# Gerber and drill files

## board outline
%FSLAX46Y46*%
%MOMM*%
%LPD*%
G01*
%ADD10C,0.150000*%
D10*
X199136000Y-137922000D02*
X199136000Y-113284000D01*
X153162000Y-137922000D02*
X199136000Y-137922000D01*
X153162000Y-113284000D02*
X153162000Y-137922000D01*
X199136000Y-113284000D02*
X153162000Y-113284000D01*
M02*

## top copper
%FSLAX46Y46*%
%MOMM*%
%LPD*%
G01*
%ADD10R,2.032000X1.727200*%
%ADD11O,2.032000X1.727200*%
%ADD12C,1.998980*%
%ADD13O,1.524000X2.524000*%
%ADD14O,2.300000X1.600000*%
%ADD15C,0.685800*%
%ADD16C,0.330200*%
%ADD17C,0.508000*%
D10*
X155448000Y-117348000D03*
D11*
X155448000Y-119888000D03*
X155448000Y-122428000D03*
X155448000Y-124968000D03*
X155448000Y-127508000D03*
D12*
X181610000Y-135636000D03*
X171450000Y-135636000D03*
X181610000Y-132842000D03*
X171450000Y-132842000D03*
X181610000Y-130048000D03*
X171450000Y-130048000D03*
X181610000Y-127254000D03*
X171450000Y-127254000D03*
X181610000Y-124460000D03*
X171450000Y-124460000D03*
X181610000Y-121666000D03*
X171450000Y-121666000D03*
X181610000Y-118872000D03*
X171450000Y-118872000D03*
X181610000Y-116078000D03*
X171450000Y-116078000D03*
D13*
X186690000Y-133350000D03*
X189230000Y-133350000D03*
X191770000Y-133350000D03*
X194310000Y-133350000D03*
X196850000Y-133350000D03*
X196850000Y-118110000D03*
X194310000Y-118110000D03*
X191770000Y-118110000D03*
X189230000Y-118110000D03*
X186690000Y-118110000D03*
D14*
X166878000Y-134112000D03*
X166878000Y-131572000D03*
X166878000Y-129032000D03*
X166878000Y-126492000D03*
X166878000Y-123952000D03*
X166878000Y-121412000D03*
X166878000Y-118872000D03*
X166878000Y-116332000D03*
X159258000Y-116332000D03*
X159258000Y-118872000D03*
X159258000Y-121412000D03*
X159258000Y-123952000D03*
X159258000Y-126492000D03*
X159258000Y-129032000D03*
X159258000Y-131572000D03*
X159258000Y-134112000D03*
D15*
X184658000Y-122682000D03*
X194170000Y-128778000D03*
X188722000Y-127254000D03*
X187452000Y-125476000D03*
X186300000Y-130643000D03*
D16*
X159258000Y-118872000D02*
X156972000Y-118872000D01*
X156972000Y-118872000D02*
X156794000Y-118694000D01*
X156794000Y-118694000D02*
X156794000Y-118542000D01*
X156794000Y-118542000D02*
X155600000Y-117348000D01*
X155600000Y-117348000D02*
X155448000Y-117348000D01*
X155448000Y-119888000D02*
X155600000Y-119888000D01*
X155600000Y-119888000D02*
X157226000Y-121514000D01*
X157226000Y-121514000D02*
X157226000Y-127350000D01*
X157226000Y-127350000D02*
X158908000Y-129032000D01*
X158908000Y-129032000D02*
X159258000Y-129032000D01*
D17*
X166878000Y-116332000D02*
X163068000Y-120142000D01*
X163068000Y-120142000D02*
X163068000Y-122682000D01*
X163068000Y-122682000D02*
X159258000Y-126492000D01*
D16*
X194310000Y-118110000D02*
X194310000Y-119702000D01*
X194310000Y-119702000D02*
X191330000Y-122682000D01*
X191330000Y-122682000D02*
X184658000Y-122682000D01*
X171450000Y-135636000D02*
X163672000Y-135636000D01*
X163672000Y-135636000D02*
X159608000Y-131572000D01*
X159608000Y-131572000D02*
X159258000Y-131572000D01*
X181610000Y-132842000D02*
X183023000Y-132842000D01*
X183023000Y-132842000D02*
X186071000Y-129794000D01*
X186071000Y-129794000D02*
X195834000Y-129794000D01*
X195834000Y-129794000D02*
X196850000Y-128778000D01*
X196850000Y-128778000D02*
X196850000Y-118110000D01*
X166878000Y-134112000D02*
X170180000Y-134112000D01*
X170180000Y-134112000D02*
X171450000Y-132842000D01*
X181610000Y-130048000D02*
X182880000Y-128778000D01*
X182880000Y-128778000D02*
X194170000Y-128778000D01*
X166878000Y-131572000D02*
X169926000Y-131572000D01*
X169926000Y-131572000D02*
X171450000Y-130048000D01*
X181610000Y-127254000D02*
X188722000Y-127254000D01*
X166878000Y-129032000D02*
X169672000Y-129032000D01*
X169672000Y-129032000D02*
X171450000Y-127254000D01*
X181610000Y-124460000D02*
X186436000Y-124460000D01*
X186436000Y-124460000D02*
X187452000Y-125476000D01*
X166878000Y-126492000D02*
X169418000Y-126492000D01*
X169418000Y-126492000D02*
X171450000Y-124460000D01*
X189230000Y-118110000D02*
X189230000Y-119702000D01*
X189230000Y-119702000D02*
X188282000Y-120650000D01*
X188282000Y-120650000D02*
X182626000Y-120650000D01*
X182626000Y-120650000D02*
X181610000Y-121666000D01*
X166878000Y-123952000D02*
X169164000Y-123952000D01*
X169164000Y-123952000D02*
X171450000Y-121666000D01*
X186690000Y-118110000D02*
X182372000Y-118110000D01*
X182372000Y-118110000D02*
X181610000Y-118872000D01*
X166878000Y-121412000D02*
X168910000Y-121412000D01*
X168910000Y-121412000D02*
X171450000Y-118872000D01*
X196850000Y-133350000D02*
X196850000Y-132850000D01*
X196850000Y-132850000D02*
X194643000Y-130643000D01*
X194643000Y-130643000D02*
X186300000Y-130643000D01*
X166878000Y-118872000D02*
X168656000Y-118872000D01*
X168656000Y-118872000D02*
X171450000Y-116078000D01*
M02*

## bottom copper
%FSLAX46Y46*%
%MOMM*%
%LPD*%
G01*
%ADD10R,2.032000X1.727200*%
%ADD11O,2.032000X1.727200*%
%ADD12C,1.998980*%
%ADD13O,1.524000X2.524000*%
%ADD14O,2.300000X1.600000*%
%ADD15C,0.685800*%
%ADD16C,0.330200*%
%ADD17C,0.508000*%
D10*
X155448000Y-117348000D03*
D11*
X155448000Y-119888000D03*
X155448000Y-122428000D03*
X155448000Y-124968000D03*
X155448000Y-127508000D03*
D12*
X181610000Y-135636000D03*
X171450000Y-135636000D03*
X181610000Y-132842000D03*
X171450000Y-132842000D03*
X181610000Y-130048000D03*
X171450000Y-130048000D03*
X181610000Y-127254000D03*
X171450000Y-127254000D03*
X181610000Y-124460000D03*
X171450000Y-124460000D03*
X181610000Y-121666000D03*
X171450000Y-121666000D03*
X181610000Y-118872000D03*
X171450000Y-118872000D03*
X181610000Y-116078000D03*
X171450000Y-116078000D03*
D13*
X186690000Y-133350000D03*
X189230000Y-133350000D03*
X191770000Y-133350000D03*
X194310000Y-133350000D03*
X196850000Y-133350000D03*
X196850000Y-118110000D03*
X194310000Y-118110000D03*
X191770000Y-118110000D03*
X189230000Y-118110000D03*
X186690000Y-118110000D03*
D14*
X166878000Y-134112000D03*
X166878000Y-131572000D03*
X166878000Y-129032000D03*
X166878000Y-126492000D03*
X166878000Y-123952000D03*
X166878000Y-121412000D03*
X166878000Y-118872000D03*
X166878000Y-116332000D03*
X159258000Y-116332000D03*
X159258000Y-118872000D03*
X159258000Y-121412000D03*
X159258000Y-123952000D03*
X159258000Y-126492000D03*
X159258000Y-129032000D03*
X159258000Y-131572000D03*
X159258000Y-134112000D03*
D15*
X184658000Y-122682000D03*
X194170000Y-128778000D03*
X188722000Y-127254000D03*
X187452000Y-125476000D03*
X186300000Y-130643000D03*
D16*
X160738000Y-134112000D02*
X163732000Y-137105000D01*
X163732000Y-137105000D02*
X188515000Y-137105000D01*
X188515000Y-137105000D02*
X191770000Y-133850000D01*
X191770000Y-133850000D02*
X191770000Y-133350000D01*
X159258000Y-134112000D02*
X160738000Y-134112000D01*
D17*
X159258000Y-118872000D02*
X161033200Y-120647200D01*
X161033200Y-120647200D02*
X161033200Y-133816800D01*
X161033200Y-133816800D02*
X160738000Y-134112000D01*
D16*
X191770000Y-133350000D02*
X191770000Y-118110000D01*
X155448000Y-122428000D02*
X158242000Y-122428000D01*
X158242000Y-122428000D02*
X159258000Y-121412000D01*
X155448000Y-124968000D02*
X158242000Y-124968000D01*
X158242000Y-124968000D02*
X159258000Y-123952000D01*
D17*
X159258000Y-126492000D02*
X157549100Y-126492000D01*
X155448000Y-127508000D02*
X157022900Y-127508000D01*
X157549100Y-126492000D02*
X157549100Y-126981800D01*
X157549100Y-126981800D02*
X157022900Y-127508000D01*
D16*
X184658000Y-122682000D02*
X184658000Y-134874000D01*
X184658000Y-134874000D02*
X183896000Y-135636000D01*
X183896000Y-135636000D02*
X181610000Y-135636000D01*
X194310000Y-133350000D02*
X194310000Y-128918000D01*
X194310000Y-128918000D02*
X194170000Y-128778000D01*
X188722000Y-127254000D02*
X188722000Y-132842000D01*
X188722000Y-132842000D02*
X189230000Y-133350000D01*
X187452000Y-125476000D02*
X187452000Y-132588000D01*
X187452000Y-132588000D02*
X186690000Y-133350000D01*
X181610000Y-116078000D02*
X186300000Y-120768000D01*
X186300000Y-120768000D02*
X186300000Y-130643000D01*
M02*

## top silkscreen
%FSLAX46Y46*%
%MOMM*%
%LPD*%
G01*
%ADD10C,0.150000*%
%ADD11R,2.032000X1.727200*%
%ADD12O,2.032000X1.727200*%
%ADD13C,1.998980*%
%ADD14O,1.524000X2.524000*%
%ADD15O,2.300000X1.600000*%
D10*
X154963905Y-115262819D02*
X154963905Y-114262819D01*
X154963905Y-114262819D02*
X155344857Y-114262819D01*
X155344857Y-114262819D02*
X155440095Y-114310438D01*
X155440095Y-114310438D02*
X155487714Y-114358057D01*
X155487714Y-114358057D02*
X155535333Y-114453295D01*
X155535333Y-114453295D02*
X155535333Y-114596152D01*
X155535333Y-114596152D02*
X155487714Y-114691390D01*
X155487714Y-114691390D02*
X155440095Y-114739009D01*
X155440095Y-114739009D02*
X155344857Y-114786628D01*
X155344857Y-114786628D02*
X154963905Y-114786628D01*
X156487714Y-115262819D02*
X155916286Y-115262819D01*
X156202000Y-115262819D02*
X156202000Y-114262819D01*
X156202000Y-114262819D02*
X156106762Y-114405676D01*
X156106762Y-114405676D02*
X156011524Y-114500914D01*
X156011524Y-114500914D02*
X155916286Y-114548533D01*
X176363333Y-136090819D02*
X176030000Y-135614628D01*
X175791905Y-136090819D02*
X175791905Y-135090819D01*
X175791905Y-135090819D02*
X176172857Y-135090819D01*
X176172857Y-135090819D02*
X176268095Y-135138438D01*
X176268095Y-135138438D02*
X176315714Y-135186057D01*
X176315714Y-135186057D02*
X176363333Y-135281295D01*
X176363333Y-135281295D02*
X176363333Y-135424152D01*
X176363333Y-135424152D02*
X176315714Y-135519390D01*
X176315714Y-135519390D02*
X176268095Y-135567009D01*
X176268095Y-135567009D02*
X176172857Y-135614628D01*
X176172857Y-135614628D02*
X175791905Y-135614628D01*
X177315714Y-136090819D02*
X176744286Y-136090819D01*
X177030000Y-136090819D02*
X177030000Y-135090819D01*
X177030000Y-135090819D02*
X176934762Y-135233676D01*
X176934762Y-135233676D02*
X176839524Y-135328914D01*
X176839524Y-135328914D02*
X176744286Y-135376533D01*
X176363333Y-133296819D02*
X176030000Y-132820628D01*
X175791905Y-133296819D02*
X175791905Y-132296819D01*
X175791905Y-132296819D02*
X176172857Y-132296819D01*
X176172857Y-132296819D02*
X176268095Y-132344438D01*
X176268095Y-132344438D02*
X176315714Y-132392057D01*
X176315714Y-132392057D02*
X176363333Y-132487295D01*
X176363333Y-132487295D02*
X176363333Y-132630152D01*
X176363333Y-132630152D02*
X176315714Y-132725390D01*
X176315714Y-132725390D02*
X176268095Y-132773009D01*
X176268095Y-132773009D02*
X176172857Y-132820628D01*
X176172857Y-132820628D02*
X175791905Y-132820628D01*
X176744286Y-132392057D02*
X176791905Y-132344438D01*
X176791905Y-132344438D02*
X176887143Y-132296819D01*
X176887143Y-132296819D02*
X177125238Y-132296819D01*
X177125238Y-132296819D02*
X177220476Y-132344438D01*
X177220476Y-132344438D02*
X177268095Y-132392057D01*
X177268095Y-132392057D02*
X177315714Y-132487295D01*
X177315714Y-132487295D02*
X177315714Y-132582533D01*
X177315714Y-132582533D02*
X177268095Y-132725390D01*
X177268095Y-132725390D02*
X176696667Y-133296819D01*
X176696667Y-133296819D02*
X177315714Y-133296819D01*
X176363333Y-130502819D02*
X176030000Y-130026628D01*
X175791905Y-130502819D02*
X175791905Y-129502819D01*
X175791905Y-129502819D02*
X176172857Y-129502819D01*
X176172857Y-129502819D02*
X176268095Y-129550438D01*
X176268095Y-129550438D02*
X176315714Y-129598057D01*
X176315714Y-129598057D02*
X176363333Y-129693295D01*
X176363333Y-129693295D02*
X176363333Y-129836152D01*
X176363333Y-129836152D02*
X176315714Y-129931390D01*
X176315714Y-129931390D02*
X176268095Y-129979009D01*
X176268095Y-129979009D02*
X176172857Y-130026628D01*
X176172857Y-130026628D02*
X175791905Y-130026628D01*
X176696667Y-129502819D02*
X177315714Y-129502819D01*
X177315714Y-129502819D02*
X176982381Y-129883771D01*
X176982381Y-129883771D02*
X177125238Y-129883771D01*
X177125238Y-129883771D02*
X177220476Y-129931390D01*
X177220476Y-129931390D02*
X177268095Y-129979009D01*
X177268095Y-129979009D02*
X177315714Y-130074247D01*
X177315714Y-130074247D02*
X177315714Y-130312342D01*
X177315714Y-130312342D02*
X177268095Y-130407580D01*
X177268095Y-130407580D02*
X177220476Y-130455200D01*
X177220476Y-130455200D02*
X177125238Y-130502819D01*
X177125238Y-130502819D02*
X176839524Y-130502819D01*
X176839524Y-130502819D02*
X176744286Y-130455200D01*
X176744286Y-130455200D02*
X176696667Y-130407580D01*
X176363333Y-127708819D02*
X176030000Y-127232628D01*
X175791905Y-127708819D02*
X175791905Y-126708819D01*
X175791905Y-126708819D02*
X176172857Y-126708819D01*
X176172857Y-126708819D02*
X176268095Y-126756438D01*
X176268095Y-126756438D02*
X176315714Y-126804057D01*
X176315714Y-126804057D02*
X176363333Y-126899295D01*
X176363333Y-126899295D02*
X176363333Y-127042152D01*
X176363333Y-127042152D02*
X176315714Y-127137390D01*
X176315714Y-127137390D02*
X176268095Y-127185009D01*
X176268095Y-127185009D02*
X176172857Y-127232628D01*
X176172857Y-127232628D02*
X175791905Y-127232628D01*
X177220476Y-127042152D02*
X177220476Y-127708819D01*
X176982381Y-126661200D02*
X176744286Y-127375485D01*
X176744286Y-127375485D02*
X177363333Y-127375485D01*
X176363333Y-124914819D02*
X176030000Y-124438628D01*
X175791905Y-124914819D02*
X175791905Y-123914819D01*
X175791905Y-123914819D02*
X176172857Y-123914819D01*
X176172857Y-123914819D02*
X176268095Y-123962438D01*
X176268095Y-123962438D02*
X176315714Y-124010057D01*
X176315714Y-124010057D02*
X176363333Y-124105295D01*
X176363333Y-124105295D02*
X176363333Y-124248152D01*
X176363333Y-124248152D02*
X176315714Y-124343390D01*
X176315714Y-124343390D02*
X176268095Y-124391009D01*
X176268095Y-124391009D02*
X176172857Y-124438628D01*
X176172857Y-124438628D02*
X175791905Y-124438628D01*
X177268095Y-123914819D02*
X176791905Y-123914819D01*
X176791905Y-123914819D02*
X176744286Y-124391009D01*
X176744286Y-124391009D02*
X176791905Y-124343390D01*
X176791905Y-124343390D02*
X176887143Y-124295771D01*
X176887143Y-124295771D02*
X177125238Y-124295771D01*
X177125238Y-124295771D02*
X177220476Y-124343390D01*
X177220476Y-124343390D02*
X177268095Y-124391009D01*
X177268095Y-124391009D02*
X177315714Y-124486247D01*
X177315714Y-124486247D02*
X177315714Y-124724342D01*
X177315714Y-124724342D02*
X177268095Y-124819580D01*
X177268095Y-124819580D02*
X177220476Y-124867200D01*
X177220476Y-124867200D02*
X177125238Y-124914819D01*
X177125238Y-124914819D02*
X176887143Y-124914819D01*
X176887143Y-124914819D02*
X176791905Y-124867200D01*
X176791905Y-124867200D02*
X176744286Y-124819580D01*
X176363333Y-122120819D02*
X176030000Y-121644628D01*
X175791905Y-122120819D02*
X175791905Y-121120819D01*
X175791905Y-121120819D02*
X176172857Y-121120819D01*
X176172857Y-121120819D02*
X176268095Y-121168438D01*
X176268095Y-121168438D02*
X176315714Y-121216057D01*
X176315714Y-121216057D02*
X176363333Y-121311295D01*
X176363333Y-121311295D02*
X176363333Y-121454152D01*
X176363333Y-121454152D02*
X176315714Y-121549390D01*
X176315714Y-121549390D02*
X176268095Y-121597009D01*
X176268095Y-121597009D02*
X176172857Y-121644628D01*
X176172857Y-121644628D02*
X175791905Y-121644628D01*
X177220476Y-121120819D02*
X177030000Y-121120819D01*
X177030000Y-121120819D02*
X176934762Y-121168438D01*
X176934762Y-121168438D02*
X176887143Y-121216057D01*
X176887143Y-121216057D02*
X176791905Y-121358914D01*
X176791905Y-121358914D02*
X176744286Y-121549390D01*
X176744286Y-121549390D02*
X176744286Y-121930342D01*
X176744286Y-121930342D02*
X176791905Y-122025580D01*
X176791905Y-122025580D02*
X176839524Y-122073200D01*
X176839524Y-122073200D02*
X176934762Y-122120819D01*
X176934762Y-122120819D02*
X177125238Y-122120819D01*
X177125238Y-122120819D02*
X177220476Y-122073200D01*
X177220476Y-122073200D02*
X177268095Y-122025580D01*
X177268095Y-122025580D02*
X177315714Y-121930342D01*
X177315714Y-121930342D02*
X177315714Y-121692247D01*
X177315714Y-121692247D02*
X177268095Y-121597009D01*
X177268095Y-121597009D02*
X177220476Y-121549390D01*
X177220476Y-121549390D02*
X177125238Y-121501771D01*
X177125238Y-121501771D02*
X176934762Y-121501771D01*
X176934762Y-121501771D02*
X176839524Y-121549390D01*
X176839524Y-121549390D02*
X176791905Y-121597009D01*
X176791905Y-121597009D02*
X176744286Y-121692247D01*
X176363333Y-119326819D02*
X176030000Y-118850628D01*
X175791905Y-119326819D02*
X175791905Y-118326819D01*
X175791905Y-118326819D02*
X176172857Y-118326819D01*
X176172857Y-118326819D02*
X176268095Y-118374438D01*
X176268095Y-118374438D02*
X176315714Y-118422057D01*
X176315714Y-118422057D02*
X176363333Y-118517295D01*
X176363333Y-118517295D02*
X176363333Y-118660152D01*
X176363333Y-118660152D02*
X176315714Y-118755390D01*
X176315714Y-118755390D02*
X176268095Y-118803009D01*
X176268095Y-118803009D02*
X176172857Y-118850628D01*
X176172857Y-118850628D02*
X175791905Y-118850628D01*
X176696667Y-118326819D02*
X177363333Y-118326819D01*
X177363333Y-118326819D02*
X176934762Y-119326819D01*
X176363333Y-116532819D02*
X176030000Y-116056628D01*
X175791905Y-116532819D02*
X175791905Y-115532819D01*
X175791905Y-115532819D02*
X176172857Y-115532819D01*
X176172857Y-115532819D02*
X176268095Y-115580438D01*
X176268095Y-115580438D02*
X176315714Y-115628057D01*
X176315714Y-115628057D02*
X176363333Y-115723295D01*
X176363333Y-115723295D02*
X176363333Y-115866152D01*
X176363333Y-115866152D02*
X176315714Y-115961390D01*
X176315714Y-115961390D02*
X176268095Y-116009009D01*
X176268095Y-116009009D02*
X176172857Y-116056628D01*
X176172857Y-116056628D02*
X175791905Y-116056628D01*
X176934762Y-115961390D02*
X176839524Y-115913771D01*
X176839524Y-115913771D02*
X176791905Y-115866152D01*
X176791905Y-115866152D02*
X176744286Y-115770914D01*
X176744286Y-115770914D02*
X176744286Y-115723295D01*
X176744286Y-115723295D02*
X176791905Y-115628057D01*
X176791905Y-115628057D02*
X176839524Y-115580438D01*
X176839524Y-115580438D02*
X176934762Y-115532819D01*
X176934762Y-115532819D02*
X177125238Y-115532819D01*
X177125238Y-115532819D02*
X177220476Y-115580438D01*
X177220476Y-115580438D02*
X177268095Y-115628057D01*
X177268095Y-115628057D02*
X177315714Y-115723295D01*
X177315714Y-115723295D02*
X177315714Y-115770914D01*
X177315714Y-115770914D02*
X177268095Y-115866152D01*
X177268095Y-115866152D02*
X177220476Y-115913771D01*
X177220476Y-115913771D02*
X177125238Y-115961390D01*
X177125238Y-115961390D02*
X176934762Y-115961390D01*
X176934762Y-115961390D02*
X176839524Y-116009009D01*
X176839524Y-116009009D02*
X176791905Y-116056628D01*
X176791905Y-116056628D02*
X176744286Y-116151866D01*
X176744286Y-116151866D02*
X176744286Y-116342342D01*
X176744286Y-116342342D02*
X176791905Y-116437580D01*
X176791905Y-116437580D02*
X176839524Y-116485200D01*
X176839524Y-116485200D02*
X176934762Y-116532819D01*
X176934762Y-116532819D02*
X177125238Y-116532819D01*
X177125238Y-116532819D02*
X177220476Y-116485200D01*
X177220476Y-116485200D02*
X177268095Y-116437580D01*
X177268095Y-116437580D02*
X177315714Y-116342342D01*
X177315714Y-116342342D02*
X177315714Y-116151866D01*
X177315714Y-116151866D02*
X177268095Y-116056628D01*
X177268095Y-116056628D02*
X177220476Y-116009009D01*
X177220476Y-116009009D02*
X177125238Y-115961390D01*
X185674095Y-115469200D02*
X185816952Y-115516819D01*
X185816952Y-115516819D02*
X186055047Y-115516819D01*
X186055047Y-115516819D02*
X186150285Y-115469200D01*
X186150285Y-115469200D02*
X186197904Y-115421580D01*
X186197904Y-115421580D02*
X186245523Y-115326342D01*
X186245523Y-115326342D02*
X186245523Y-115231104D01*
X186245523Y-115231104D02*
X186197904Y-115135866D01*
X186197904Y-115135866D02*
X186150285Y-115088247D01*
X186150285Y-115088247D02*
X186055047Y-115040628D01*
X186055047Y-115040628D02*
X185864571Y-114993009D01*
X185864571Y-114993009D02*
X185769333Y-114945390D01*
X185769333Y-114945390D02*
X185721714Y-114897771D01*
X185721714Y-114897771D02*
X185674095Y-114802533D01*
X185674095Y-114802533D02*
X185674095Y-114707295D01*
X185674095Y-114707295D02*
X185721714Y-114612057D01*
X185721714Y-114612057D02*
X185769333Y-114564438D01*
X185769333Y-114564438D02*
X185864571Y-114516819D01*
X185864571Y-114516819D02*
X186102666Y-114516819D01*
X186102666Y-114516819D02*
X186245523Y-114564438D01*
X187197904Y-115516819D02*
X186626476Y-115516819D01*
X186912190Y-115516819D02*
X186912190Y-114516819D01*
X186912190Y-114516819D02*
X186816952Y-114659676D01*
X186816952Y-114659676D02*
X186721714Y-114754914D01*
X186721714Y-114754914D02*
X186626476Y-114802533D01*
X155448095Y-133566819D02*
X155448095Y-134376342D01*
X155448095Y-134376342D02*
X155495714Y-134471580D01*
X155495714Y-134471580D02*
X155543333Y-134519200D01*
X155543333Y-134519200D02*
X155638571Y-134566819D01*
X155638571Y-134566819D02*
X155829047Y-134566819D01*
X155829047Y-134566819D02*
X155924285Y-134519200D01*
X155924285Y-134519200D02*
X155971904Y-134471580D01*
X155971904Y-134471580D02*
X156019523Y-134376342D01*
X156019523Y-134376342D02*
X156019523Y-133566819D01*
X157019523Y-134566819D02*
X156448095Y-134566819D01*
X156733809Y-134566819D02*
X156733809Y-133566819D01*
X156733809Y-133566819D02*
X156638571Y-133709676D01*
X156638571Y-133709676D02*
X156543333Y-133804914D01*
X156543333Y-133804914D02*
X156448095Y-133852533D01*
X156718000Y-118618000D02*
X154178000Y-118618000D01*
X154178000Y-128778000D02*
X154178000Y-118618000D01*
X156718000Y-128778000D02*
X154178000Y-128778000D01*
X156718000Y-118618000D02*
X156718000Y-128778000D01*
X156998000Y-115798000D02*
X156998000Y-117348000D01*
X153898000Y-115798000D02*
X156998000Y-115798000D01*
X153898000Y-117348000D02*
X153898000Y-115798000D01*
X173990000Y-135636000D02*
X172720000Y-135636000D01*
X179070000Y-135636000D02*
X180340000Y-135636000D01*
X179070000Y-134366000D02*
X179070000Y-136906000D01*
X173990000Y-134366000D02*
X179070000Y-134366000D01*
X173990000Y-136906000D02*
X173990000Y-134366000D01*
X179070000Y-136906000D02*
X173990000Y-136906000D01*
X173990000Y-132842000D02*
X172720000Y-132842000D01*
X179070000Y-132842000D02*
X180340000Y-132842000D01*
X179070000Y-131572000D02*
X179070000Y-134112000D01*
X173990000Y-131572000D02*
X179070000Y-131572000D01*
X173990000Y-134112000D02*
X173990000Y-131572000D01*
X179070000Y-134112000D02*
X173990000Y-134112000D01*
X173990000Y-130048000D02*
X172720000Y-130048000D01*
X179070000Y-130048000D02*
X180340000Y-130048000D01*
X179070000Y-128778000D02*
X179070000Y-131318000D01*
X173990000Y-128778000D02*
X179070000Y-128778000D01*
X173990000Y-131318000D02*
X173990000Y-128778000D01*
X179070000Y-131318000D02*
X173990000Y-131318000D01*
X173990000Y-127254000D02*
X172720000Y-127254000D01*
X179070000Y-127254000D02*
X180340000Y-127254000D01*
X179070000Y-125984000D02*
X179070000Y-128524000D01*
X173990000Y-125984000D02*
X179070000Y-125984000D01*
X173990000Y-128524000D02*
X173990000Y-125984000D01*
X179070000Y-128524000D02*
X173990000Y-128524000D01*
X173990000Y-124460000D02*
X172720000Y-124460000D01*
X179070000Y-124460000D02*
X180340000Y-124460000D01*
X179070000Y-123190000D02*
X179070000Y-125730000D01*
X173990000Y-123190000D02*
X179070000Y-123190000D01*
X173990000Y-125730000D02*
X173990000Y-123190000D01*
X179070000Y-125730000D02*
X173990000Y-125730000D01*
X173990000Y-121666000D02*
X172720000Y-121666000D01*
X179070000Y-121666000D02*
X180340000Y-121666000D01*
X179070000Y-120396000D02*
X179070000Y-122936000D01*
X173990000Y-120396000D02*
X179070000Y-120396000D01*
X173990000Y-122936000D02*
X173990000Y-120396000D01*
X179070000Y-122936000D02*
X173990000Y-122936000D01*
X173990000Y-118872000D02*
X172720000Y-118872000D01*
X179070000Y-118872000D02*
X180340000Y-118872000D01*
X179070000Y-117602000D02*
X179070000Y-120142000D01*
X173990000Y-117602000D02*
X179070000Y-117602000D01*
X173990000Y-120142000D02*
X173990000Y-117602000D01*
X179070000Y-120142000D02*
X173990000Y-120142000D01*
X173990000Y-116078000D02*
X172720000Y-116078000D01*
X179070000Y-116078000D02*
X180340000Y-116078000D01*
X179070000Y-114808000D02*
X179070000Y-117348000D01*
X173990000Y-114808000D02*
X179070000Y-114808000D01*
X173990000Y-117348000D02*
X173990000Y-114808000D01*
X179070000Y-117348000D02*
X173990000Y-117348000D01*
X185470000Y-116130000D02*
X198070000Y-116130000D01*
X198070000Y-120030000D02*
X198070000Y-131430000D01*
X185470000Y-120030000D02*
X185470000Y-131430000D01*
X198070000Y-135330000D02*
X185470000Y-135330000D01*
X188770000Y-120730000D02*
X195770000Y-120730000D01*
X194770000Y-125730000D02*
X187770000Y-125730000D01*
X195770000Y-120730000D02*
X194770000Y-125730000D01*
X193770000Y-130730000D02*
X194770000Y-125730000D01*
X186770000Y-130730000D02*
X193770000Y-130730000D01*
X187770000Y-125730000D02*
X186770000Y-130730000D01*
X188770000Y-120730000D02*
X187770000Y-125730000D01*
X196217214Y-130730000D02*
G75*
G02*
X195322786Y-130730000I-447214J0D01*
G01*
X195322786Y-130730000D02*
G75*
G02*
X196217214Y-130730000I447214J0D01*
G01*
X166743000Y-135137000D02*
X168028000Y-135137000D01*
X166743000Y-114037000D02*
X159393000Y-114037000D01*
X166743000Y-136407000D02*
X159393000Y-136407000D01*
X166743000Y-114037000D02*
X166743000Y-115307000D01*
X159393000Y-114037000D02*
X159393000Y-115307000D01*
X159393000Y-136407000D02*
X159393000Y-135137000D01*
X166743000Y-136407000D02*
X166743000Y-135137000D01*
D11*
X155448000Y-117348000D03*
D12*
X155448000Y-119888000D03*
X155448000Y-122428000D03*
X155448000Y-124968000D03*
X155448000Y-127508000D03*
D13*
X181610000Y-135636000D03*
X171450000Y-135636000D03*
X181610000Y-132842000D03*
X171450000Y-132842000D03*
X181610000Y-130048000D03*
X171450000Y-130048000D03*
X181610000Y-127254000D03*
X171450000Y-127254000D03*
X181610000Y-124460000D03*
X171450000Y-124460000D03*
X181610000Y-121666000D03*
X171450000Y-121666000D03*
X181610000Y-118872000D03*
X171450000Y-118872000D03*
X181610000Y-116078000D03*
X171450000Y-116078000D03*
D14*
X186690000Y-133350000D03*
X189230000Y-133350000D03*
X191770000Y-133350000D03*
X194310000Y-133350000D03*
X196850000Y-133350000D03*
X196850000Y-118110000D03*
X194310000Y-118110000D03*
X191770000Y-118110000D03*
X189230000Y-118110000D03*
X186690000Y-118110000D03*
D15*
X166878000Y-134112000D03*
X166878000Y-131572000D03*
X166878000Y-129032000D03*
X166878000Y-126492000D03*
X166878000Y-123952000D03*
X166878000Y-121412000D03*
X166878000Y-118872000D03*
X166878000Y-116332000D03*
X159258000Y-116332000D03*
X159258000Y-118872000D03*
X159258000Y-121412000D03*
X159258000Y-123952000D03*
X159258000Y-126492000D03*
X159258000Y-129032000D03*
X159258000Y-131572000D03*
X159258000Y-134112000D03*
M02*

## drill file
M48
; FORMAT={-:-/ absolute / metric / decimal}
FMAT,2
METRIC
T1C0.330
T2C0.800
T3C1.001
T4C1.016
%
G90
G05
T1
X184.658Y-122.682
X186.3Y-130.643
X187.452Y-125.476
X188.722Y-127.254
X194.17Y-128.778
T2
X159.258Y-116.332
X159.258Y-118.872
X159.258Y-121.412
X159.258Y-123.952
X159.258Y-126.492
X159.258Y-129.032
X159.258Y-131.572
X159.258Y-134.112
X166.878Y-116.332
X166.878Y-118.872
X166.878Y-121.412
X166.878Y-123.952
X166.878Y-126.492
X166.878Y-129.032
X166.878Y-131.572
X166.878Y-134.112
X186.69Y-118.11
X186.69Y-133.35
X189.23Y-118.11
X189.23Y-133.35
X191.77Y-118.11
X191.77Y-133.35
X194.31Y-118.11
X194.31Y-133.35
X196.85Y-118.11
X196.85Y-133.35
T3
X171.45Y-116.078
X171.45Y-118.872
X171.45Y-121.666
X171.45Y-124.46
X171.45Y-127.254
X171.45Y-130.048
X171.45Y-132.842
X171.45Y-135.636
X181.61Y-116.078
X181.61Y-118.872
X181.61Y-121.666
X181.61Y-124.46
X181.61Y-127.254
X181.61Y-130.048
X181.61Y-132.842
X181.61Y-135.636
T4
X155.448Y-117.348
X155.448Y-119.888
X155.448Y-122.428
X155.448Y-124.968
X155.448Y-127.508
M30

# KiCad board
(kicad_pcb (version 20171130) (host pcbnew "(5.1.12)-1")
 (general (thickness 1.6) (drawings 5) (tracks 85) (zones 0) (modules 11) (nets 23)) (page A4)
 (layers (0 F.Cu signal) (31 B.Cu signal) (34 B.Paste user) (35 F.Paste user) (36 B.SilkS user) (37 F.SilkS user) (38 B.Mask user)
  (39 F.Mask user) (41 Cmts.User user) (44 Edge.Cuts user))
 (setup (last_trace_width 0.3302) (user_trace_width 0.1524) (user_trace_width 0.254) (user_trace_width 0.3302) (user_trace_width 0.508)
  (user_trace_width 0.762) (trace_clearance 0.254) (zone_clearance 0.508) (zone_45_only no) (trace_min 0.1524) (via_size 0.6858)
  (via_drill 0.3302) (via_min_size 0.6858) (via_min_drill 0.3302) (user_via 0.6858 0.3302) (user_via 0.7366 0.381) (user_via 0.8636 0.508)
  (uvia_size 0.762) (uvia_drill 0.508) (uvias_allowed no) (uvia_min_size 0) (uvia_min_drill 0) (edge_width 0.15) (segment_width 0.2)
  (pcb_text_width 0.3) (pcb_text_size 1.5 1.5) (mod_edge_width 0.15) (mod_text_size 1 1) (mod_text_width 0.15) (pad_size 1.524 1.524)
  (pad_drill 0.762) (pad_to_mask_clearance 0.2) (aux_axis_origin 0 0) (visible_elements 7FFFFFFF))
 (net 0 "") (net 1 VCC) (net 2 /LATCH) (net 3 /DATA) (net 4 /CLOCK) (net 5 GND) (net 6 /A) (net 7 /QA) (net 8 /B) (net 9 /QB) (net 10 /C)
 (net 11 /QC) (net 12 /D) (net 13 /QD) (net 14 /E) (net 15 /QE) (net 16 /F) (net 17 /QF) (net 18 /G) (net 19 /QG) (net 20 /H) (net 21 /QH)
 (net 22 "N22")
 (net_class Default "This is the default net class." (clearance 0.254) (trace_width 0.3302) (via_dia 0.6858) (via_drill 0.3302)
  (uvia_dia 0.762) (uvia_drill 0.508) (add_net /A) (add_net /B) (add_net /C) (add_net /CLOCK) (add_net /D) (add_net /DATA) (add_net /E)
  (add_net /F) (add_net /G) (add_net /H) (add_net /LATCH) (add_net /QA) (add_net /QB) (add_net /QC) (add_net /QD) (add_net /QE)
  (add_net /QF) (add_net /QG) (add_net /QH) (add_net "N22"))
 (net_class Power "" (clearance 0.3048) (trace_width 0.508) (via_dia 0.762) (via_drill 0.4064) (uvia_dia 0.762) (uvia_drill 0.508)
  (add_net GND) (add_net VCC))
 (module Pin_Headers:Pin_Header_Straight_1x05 (layer F.Cu) (at 155.448 117.348)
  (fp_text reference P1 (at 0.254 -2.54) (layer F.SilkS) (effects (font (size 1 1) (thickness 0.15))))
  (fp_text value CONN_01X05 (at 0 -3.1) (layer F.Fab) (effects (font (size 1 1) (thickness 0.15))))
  (fp_line (start 1.27 1.27) (end -1.27 1.27) (layer F.SilkS) (width 0.15))
  (fp_line (start -1.27 11.43) (end -1.27 1.27) (layer F.SilkS) (width 0.15))
  (fp_line (start 1.27 11.43) (end -1.27 11.43) (layer F.SilkS) (width 0.15))
  (fp_line (start 1.27 1.27) (end 1.27 11.43) (layer F.SilkS) (width 0.15))
  (fp_line (start 1.55 -1.55) (end 1.55 0) (layer F.SilkS) (width 0.15))
  (fp_line (start -1.55 -1.55) (end 1.55 -1.55) (layer F.SilkS) (width 0.15))
  (fp_line (start -1.55 0) (end -1.55 -1.55) (layer F.SilkS) (width 0.15))
  (pad 1 thru_hole rect (at 0 0) (size 2.032 1.7272) (drill 1.016) (layers *.Cu *.Mask F.SilkS) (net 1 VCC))
  (pad 2 thru_hole oval (at 0 2.54) (size 2.032 1.7272) (drill 1.016) (layers *.Cu *.Mask F.SilkS) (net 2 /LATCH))
  (pad 3 thru_hole oval (at 0 5.08) (size 2.032 1.7272) (drill 1.016) (layers *.Cu *.Mask F.SilkS) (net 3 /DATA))
  (pad 4 thru_hole oval (at 0 7.62) (size 2.032 1.7272) (drill 1.016) (layers *.Cu *.Mask F.SilkS) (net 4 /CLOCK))
  (pad 5 thru_hole oval (at 0 10.16) (size 2.032 1.7272) (drill 1.016) (layers *.Cu *.Mask F.SilkS) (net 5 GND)))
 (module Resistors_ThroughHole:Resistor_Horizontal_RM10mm (layer F.Cu) (at 176.53 135.636 180)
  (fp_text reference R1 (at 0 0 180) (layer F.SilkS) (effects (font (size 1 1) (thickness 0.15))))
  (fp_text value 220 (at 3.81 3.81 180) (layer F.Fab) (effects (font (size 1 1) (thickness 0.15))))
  (fp_line (start 2.54 0) (end 3.81 0) (layer F.SilkS) (width 0.15))
  (fp_line (start -2.54 0) (end -3.81 0) (layer F.SilkS) (width 0.15))
  (fp_line (start -2.54 1.27) (end -2.54 -1.27) (layer F.SilkS) (width 0.15))
  (fp_line (start 2.54 1.27) (end -2.54 1.27) (layer F.SilkS) (width 0.15))
  (fp_line (start 2.54 -1.27) (end 2.54 1.27) (layer F.SilkS) (width 0.15))
  (fp_line (start -2.54 -1.27) (end 2.54 -1.27) (layer F.SilkS) (width 0.15))
  (pad 1 thru_hole circle (at -5.08 0 180) (size 1.99898 1.99898) (drill 1.00076) (layers *.Cu *.SilkS *.Mask) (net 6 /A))
  (pad 2 thru_hole circle (at 5.08 0 180) (size 1.99898 1.99898) (drill 1.00076) (layers *.Cu *.SilkS *.Mask) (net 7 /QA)))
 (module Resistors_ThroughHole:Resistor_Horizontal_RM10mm (layer F.Cu) (at 176.53 132.842 180)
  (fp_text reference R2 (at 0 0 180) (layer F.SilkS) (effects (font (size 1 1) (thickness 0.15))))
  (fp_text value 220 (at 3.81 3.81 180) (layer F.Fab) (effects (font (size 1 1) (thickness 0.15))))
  (fp_line (start 2.54 0) (end 3.81 0) (layer F.SilkS) (width 0.15))
  (fp_line (start -2.54 0) (end -3.81 0) (layer F.SilkS) (width 0.15))
  (fp_line (start -2.54 1.27) (end -2.54 -1.27) (layer F.SilkS) (width 0.15))
  (fp_line (start 2.54 1.27) (end -2.54 1.27) (layer F.SilkS) (width 0.15))
  (fp_line (start 2.54 -1.27) (end 2.54 1.27) (layer F.SilkS) (width 0.15))
  (fp_line (start -2.54 -1.27) (end 2.54 -1.27) (layer F.SilkS) (width 0.15))
  (pad 1 thru_hole circle (at -5.08 0 180) (size 1.99898 1.99898) (drill 1.00076) (layers *.Cu *.SilkS *.Mask) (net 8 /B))
  (pad 2 thru_hole circle (at 5.08 0 180) (size 1.99898 1.99898) (drill 1.00076) (layers *.Cu *.SilkS *.Mask) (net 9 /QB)))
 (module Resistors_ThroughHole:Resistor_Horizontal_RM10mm (layer F.Cu) (at 176.53 130.048 180)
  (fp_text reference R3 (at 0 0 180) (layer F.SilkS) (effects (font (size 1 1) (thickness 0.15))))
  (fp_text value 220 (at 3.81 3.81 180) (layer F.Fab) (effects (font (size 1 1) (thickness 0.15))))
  (fp_line (start 2.54 0) (end 3.81 0) (layer F.SilkS) (width 0.15))
  (fp_line (start -2.54 0) (end -3.81 0) (layer F.SilkS) (width 0.15))
  (fp_line (start -2.54 1.27) (end -2.54 -1.27) (layer F.SilkS) (width 0.15))
  (fp_line (start 2.54 1.27) (end -2.54 1.27) (layer F.SilkS) (width 0.15))
  (fp_line (start 2.54 -1.27) (end 2.54 1.27) (layer F.SilkS) (width 0.15))
  (fp_line (start -2.54 -1.27) (end 2.54 -1.27) (layer F.SilkS) (width 0.15))
  (pad 1 thru_hole circle (at -5.08 0 180) (size 1.99898 1.99898) (drill 1.00076) (layers *.Cu *.SilkS *.Mask) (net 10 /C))
  (pad 2 thru_hole circle (at 5.08 0 180) (size 1.99898 1.99898) (drill 1.00076) (layers *.Cu *.SilkS *.Mask) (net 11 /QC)))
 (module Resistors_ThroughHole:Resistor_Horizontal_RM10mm (layer F.Cu) (at 176.53 127.254 180)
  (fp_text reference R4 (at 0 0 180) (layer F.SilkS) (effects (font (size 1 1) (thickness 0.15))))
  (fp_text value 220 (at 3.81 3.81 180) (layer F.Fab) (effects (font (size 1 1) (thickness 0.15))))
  (fp_line (start 2.54 0) (end 3.81 0) (layer F.SilkS) (width 0.15))
  (fp_line (start -2.54 0) (end -3.81 0) (layer F.SilkS) (width 0.15))
  (fp_line (start -2.54 1.27) (end -2.54 -1.27) (layer F.SilkS) (width 0.15))
  (fp_line (start 2.54 1.27) (end -2.54 1.27) (layer F.SilkS) (width 0.15))
  (fp_line (start 2.54 -1.27) (end 2.54 1.27) (layer F.SilkS) (width 0.15))
  (fp_line (start -2.54 -1.27) (end 2.54 -1.27) (layer F.SilkS) (width 0.15))
  (pad 1 thru_hole circle (at -5.08 0 180) (size 1.99898 1.99898) (drill 1.00076) (layers *.Cu *.SilkS *.Mask) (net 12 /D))
  (pad 2 thru_hole circle (at 5.08 0 180) (size 1.99898 1.99898) (drill 1.00076) (layers *.Cu *.SilkS *.Mask) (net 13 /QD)))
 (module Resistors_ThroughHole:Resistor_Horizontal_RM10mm (layer F.Cu) (at 176.53 124.46 180)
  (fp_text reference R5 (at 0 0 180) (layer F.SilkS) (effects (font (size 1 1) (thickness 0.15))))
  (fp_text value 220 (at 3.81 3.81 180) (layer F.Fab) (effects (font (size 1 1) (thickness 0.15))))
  (fp_line (start 2.54 0) (end 3.81 0) (layer F.SilkS) (width 0.15))
  (fp_line (start -2.54 0) (end -3.81 0) (layer F.SilkS) (width 0.15))
  (fp_line (start -2.54 1.27) (end -2.54 -1.27) (layer F.SilkS) (width 0.15))
  (fp_line (start 2.54 1.27) (end -2.54 1.27) (layer F.SilkS) (width 0.15))
  (fp_line (start 2.54 -1.27) (end 2.54 1.27) (layer F.SilkS) (width 0.15))
  (fp_line (start -2.54 -1.27) (end 2.54 -1.27) (layer F.SilkS) (width 0.15))
  (pad 1 thru_hole circle (at -5.08 0 180) (size 1.99898 1.99898) (drill 1.00076) (layers *.Cu *.SilkS *.Mask) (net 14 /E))
  (pad 2 thru_hole circle (at 5.08 0 180) (size 1.99898 1.99898) (drill 1.00076) (layers *.Cu *.SilkS *.Mask) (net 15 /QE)))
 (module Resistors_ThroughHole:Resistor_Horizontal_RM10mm (layer F.Cu) (at 176.53 121.666 180)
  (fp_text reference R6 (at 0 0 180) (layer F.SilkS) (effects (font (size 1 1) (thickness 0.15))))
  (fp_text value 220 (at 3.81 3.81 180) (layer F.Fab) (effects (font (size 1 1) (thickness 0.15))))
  (fp_line (start 2.54 0) (end 3.81 0) (layer F.SilkS) (width 0.15))
  (fp_line (start -2.54 0) (end -3.81 0) (layer F.SilkS) (width 0.15))
  (fp_line (start -2.54 1.27) (end -2.54 -1.27) (layer F.SilkS) (width 0.15))
  (fp_line (start 2.54 1.27) (end -2.54 1.27) (layer F.SilkS) (width 0.15))
  (fp_line (start 2.54 -1.27) (end 2.54 1.27) (layer F.SilkS) (width 0.15))
  (fp_line (start -2.54 -1.27) (end 2.54 -1.27) (layer F.SilkS) (width 0.15))
  (pad 1 thru_hole circle (at -5.08 0 180) (size 1.99898 1.99898) (drill 1.00076) (layers *.Cu *.SilkS *.Mask) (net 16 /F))
  (pad 2 thru_hole circle (at 5.08 0 180) (size 1.99898 1.99898) (drill 1.00076) (layers *.Cu *.SilkS *.Mask) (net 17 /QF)))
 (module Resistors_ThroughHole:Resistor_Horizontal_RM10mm (layer F.Cu) (at 176.53 118.872 180)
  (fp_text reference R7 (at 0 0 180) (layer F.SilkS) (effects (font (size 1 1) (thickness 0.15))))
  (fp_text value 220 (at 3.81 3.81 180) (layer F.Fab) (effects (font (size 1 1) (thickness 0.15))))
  (fp_line (start 2.54 0) (end 3.81 0) (layer F.SilkS) (width 0.15))
  (fp_line (start -2.54 0) (end -3.81 0) (layer F.SilkS) (width 0.15))
  (fp_line (start -2.54 1.27) (end -2.54 -1.27) (layer F.SilkS) (width 0.15))
  (fp_line (start 2.54 1.27) (end -2.54 1.27) (layer F.SilkS) (width 0.15))
  (fp_line (start 2.54 -1.27) (end 2.54 1.27) (layer F.SilkS) (width 0.15))
  (fp_line (start -2.54 -1.27) (end 2.54 -1.27) (layer F.SilkS) (width 0.15))
  (pad 1 thru_hole circle (at -5.08 0 180) (size 1.99898 1.99898) (drill 1.00076) (layers *.Cu *.SilkS *.Mask) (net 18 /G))
  (pad 2 thru_hole circle (at 5.08 0 180) (size 1.99898 1.99898) (drill 1.00076) (layers *.Cu *.SilkS *.Mask) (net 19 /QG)))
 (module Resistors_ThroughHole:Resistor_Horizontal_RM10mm (layer F.Cu) (at 176.53 116.078 180)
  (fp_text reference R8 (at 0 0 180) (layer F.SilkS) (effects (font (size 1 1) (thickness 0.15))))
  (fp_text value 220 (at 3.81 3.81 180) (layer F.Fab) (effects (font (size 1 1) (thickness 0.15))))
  (fp_line (start 2.54 0) (end 3.81 0) (layer F.SilkS) (width 0.15))
  (fp_line (start -2.54 0) (end -3.81 0) (layer F.SilkS) (width 0.15))
  (fp_line (start -2.54 1.27) (end -2.54 -1.27) (layer F.SilkS) (width 0.15))
  (fp_line (start 2.54 1.27) (end -2.54 1.27) (layer F.SilkS) (width 0.15))
  (fp_line (start 2.54 -1.27) (end 2.54 1.27) (layer F.SilkS) (width 0.15))
  (fp_line (start -2.54 -1.27) (end 2.54 -1.27) (layer F.SilkS) (width 0.15))
  (pad 1 thru_hole circle (at -5.08 0 180) (size 1.99898 1.99898) (drill 1.00076) (layers *.Cu *.SilkS *.Mask) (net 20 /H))
  (pad 2 thru_hole circle (at 5.08 0 180) (size 1.99898 1.99898) (drill 1.00076) (layers *.Cu *.SilkS *.Mask) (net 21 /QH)))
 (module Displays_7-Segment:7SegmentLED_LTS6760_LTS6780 (layer F.Cu) (at 191.77 125.73)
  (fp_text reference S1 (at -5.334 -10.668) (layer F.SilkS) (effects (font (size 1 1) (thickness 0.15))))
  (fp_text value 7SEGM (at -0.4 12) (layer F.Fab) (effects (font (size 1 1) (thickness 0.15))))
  (fp_line (start -6.3 -9.6) (end 6.3 -9.6) (layer F.SilkS) (width 0.15))
  (fp_line (start 6.3 -5.7) (end 6.3 5.7) (layer F.SilkS) (width 0.15))
  (fp_line (start -6.3 -5.7) (end -6.3 5.7) (layer F.SilkS) (width 0.15))
  (fp_line (start 6.3 9.6) (end -6.3 9.6) (layer F.SilkS) (width 0.15))
  (fp_line (start -3 -5) (end 4 -5) (layer F.SilkS) (width 0.15))
  (fp_line (start 3 0) (end -4 0) (layer F.SilkS) (width 0.15))
  (fp_line (start 4 -5) (end 3 0) (layer F.SilkS) (width 0.15)) (fp_line (start 2 5) (end 3 0) (layer F.SilkS) (width 0.15))
  (fp_line (start -5 5) (end 2 5) (layer F.SilkS) (width 0.15))
  (fp_line (start -4 0) (end -5 5) (layer F.SilkS) (width 0.15))
  (fp_line (start -3 -5) (end -4 0) (layer F.SilkS) (width 0.15))
  (fp_circle (center 4 5) (end 4.4 5.2) (layer F.SilkS) (width 0.15))
  (pad 1 thru_hole oval (at -5.08 7.62) (size 1.524 2.524) (drill 0.8) (layers *.Cu *.Mask F.SilkS) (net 14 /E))
  (pad 2 thru_hole oval (at -2.54 7.62) (size 1.524 2.524) (drill 0.8) (layers *.Cu *.Mask F.SilkS) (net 12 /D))
  (pad 3 thru_hole oval (at 0 7.62) (size 1.524 2.524) (drill 0.8) (layers *.Cu *.Mask F.SilkS) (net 1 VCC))
  (pad 4 thru_hole oval (at 2.54 7.62) (size 1.524 2.524) (drill 0.8) (layers *.Cu *.Mask F.SilkS) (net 10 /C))
  (pad 5 thru_hole oval (at 5.08 7.62) (size 1.524 2.524) (drill 0.8) (layers *.Cu *.Mask F.SilkS) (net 20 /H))
  (pad 6 thru_hole oval (at 5.08 -7.62) (size 1.524 2.524) (drill 0.8) (layers *.Cu *.Mask F.SilkS) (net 8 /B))
  (pad 7 thru_hole oval (at 2.54 -7.62) (size 1.524 2.524) (drill 0.8) (layers *.Cu *.Mask F.SilkS) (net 6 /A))
  (pad 8 thru_hole oval (at 0 -7.62) (size 1.524 2.524) (drill 0.8) (layers *.Cu *.Mask F.SilkS) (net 1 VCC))
  (pad 9 thru_hole oval (at -2.54 -7.62) (size 1.524 2.524) (drill 0.8) (layers *.Cu *.Mask F.SilkS) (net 16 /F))
  (pad 10 thru_hole oval (at -5.08 -7.62) (size 1.524 2.524) (drill 0.8) (layers *.Cu *.Mask F.SilkS) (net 18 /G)))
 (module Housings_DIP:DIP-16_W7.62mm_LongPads (layer F.Cu) (at 166.878 134.112 180)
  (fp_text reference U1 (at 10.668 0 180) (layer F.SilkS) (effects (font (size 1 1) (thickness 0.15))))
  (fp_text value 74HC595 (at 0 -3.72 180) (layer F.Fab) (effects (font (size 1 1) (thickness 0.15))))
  (fp_line (start 0.135 -1.025) (end -1.15 -1.025) (layer F.SilkS) (width 0.15))
  (fp_line (start 0.135 20.075) (end 7.485 20.075) (layer F.SilkS) (width 0.15))
  (fp_line (start 0.135 -2.295) (end 7.485 -2.295) (layer F.SilkS) (width 0.15))
  (fp_line (start 0.135 20.075) (end 0.135 18.805) (layer F.SilkS) (width 0.15))
  (fp_line (start 7.485 20.075) (end 7.485 18.805) (layer F.SilkS) (width 0.15))
  (fp_line (start 7.485 -2.295) (end 7.485 -1.025) (layer F.SilkS) (width 0.15))
  (fp_line (start 0.135 -2.295) (end 0.135 -1.025) (layer F.SilkS) (width 0.15))
  (pad 1 thru_hole oval (at 0 0 180) (size 2.3 1.6) (drill 0.8) (layers *.Cu *.Mask F.SilkS) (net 9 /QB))
  (pad 2 thru_hole oval (at 0 2.54 180) (size 2.3 1.6) (drill 0.8) (layers *.Cu *.Mask F.SilkS) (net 11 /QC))
  (pad 3 thru_hole oval (at 0 5.08 180) (size 2.3 1.6) (drill 0.8) (layers *.Cu *.Mask F.SilkS) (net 13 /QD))
  (pad 4 thru_hole oval (at 0 7.62 180) (size 2.3 1.6) (drill 0.8) (layers *.Cu *.Mask F.SilkS) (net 15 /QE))
  (pad 5 thru_hole oval (at 0 10.16 180) (size 2.3 1.6) (drill 0.8) (layers *.Cu *.Mask F.SilkS) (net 17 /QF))
  (pad 6 thru_hole oval (at 0 12.7 180) (size 2.3 1.6) (drill 0.8) (layers *.Cu *.Mask F.SilkS) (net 19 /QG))
  (pad 7 thru_hole oval (at 0 15.24 180) (size 2.3 1.6) (drill 0.8) (layers *.Cu *.Mask F.SilkS) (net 21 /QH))
  (pad 8 thru_hole oval (at 0 17.78 180) (size 2.3 1.6) (drill 0.8) (layers *.Cu *.Mask F.SilkS) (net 5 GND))
  (pad 9 thru_hole oval (at 7.62 17.78 180) (size 2.3 1.6) (drill 0.8) (layers *.Cu *.Mask F.SilkS) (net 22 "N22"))
  (pad 10 thru_hole oval (at 7.62 15.24 180) (size 2.3 1.6) (drill 0.8) (layers *.Cu *.Mask F.SilkS) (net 1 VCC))
  (pad 11 thru_hole oval (at 7.62 12.7 180) (size 2.3 1.6) (drill 0.8) (layers *.Cu *.Mask F.SilkS) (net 3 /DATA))
  (pad 12 thru_hole oval (at 7.62 10.16 180) (size 2.3 1.6) (drill 0.8) (layers *.Cu *.Mask F.SilkS) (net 4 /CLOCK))
  (pad 13 thru_hole oval (at 7.62 7.62 180) (size 2.3 1.6) (drill 0.8) (layers *.Cu *.Mask F.SilkS) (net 5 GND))
  (pad 14 thru_hole oval (at 7.62 5.08 180) (size 2.3 1.6) (drill 0.8) (layers *.Cu *.Mask F.SilkS) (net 2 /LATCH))
  (pad 15 thru_hole oval (at 7.62 2.54 180) (size 2.3 1.6) (drill 0.8) (layers *.Cu *.Mask F.SilkS) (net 7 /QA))
  (pad 16 thru_hole oval (at 7.62 0 180) (size 2.3 1.6) (drill 0.8) (layers *.Cu *.Mask F.SilkS) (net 1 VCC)))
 (gr_line (start 199.136 137.922) (end 199.136 113.284) (angle 90) (layer Edge.Cuts) (width 0.15))
 (gr_line (start 153.162 137.922) (end 199.136 137.922) (angle 90) (layer Edge.Cuts) (width 0.15))
 (gr_line (start 153.162 113.284) (end 153.162 137.922) (angle 90) (layer Edge.Cuts) (width 0.15))
 (gr_line (start 199.136 113.284) (end 153.162 113.284) (angle 90) (layer Edge.Cuts) (width 0.15))
 (segment (start 160.738 134.112) (end 163.732 137.105) (width 0.3302) (layer B.Cu) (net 1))
 (segment (start 163.732 137.105) (end 188.515 137.105) (width 0.3302) (layer B.Cu) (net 1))
 (segment (start 188.515 137.105) (end 191.77 133.85) (width 0.3302) (layer B.Cu) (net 1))
 (segment (start 191.77 133.85) (end 191.77 133.35) (width 0.3302) (layer B.Cu) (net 1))
 (segment (start 159.258 134.112) (end 160.738 134.112) (width 0.3302) (layer B.Cu) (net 1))
 (segment (start 159.258 118.872) (end 161.0332 120.6472) (width 0.508) (layer B.Cu) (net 1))
 (segment (start 161.0332 120.6472) (end 161.0332 133.8168) (width 0.508) (layer B.Cu) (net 1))
 (segment (start 161.0332 133.8168) (end 160.738 134.112) (width 0.508) (layer B.Cu) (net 1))
 (segment (start 159.258 118.872) (end 156.972 118.872) (width 0.3302) (layer F.Cu) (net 1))
 (segment (start 156.972 118.872) (end 156.794 118.694) (width 0.3302) (layer F.Cu) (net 1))
 (segment (start 156.794 118.694) (end 156.794 118.542) (width 0.3302) (layer F.Cu) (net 1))
 (segment (start 156.794 118.542) (end 155.6 117.348) (width 0.3302) (layer F.Cu) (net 1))
 (segment (start 155.6 117.348) (end 155.448 117.348) (width 0.3302) (layer F.Cu) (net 1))
 (segment (start 191.77 133.35) (end 191.77 118.11) (width 0.3302) (layer B.Cu) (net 1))
 (segment (start 155.448 119.888) (end 155.6 119.888) (width 0.3302) (layer F.Cu) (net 2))
 (segment (start 155.6 119.888) (end 157.226 121.514) (width 0.3302) (layer F.Cu) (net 2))
 (segment (start 157.226 121.514) (end 157.226 127.35) (width 0.3302) (layer F.Cu) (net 2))
 (segment (start 157.226 127.35) (end 158.908 129.032) (width 0.3302) (layer F.Cu) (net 2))
 (segment (start 158.908 129.032) (end 159.258 129.032) (width 0.3302) (layer F.Cu) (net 2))
 (segment (start 155.448 122.428) (end 158.242 122.428) (width 0.3302) (layer B.Cu) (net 3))
 (segment (start 158.242 122.428) (end 159.258 121.412) (width 0.3302) (layer B.Cu) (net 3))
 (segment (start 155.448 124.968) (end 158.242 124.968) (width 0.3302) (layer B.Cu) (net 4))
 (segment (start 158.242 124.968) (end 159.258 123.952) (width 0.3302) (layer B.Cu) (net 4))
 (segment (start 166.878 116.332) (end 163.068 120.142) (width 0.508) (layer F.Cu) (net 5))
 (segment (start 163.068 120.142) (end 163.068 122.682) (width 0.508) (layer F.Cu) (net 5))
 (segment (start 163.068 122.682) (end 159.258 126.492) (width 0.508) (layer F.Cu) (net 5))
 (segment (start 159.258 126.492) (end 157.5491 126.492) (width 0.508) (layer B.Cu) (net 5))
 (segment (start 155.448 127.508) (end 157.0229 127.508) (width 0.508) (layer B.Cu) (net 5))
 (segment (start 157.5491 126.492) (end 157.5491 126.9818) (width 0.508) (layer B.Cu) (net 5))
 (segment (start 157.5491 126.9818) (end 157.0229 127.508) (width 0.508) (layer B.Cu) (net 5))
 (segment (start 194.31 118.11) (end 194.31 119.702) (width 0.3302) (layer F.Cu) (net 6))
 (segment (start 194.31 119.702) (end 191.33 122.682) (width 0.3302) (layer F.Cu) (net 6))
 (segment (start 191.33 122.682) (end 184.658 122.682) (width 0.3302) (layer F.Cu) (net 6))
 (segment (start 184.658 122.682) (end 184.658 134.874) (width 0.3302) (layer B.Cu) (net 6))
 (segment (start 184.658 134.874) (end 183.896 135.636) (width 0.3302) (layer B.Cu) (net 6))
 (segment (start 183.896 135.636) (end 181.61 135.636) (width 0.3302) (layer B.Cu) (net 6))
 (via (at 184.658 122.682) (size 0.6858) (layers F.Cu B.Cu) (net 6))
 (segment (start 171.45 135.636) (end 163.672 135.636) (width 0.3302) (layer F.Cu) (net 7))
 (segment (start 163.672 135.636) (end 159.608 131.572) (width 0.3302) (layer F.Cu) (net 7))
 (segment (start 159.608 131.572) (end 159.258 131.572) (width 0.3302) (layer F.Cu) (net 7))
 (segment (start 181.61 132.842) (end 183.023 132.842) (width 0.3302) (layer F.Cu) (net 8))
 (segment (start 183.023 132.842) (end 186.071 129.794) (width 0.3302) (layer F.Cu) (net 8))
 (segment (start 186.071 129.794) (end 195.834 129.794) (width 0.3302) (layer F.Cu) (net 8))
 (segment (start 195.834 129.794) (end 196.85 128.778) (width 0.3302) (layer F.Cu) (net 8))
 (segment (start 196.85 128.778) (end 196.85 118.11) (width 0.3302) (layer F.Cu) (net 8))
 (segment (start 166.878 134.112) (end 170.18 134.112) (width 0.3302) (layer F.Cu) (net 9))
 (segment (start 170.18 134.112) (end 171.45 132.842) (width 0.3302) (layer F.Cu) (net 9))
 (segment (start 181.61 130.048) (end 182.88 128.778) (width 0.3302) (layer F.Cu) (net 10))
 (segment (start 182.88 128.778) (end 194.17 128.778) (width 0.3302) (layer F.Cu) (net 10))
 (segment (start 194.31 133.35) (end 194.31 128.918) (width 0.3302) (layer B.Cu) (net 10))
 (segment (start 194.31 128.918) (end 194.17 128.778) (width 0.3302) (layer B.Cu) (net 10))
 (via (at 194.17 128.778) (size 0.6858) (layers F.Cu B.Cu) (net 10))
 (segment (start 166.878 131.572) (end 169.926 131.572) (width 0.3302) (layer F.Cu) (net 11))
 (segment (start 169.926 131.572) (end 171.45 130.048) (width 0.3302) (layer F.Cu) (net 11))
 (segment (start 181.61 127.254) (end 188.722 127.254) (width 0.3302) (layer F.Cu) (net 12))
 (segment (start 188.722 127.254) (end 188.722 132.842) (width 0.3302) (layer B.Cu) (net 12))
 (segment (start 188.722 132.842) (end 189.23 133.35) (width 0.3302) (layer B.Cu) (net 12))
 (via (at 188.722 127.254) (size 0.6858) (layers F.Cu B.Cu) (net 12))
 (segment (start 166.878 129.032) (end 169.672 129.032) (width 0.3302) (layer F.Cu) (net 13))
 (segment (start 169.672 129.032) (end 171.45 127.254) (width 0.3302) (layer F.Cu) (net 13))
 (segment (start 181.61 124.46) (end 186.436 124.46) (width 0.3302) (layer F.Cu) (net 14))
 (segment (start 186.436 124.46) (end 187.452 125.476) (width 0.3302) (layer F.Cu) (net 14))
 (segment (start 187.452 125.476) (end 187.452 132.588) (width 0.3302) (layer B.Cu) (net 14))
 (segment (start 187.452 132.588) (end 186.69 133.35) (width 0.3302) (layer B.Cu) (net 14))
 (via (at 187.452 125.476) (size 0.6858) (layers F.Cu B.Cu) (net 14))
 (segment (start 166.878 126.492) (end 169.418 126.492) (width 0.3302) (layer F.Cu) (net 15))
 (segment (start 169.418 126.492) (end 171.45 124.46) (width 0.3302) (layer F.Cu) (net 15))
 (segment (start 189.23 118.11) (end 189.23 119.702) (width 0.3302) (layer F.Cu) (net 16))
 (segment (start 189.23 119.702) (end 188.282 120.65) (width 0.3302) (layer F.Cu) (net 16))
 (segment (start 188.282 120.65) (end 182.626 120.65) (width 0.3302) (layer F.Cu) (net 16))
 (segment (start 182.626 120.65) (end 181.61 121.666) (width 0.3302) (layer F.Cu) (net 16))
 (segment (start 166.878 123.952) (end 169.164 123.952) (width 0.3302) (layer F.Cu) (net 17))
 (segment (start 169.164 123.952) (end 171.45 121.666) (width 0.3302) (layer F.Cu) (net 17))
 (segment (start 186.69 118.11) (end 182.372 118.11) (width 0.3302) (layer F.Cu) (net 18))
 (segment (start 182.372 118.11) (end 181.61 118.872) (width 0.3302) (layer F.Cu) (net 18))
 (segment (start 166.878 121.412) (end 168.91 121.412) (width 0.3302) (layer F.Cu) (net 19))
 (segment (start 168.91 121.412) (end 171.45 118.872) (width 0.3302) (layer F.Cu) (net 19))
 (segment (start 196.85 133.35) (end 196.85 132.85) (width 0.3302) (layer F.Cu) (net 20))
 (segment (start 196.85 132.85) (end 194.643 130.643) (width 0.3302) (layer F.Cu) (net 20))
 (segment (start 194.643 130.643) (end 186.3 130.643) (width 0.3302) (layer F.Cu) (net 20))
 (segment (start 181.61 116.078) (end 186.3 120.768) (width 0.3302) (layer B.Cu) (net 20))
 (segment (start 186.3 120.768) (end 186.3 130.643) (width 0.3302) (layer B.Cu) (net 20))
 (via (at 186.3 130.643) (size 0.6858) (layers F.Cu B.Cu) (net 20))
 (segment (start 166.878 118.872) (end 168.656 118.872) (width 0.3302) (layer F.Cu) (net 21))
 (segment (start 168.656 118.872) (end 171.45 116.078) (width 0.3302) (layer F.Cu) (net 21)))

